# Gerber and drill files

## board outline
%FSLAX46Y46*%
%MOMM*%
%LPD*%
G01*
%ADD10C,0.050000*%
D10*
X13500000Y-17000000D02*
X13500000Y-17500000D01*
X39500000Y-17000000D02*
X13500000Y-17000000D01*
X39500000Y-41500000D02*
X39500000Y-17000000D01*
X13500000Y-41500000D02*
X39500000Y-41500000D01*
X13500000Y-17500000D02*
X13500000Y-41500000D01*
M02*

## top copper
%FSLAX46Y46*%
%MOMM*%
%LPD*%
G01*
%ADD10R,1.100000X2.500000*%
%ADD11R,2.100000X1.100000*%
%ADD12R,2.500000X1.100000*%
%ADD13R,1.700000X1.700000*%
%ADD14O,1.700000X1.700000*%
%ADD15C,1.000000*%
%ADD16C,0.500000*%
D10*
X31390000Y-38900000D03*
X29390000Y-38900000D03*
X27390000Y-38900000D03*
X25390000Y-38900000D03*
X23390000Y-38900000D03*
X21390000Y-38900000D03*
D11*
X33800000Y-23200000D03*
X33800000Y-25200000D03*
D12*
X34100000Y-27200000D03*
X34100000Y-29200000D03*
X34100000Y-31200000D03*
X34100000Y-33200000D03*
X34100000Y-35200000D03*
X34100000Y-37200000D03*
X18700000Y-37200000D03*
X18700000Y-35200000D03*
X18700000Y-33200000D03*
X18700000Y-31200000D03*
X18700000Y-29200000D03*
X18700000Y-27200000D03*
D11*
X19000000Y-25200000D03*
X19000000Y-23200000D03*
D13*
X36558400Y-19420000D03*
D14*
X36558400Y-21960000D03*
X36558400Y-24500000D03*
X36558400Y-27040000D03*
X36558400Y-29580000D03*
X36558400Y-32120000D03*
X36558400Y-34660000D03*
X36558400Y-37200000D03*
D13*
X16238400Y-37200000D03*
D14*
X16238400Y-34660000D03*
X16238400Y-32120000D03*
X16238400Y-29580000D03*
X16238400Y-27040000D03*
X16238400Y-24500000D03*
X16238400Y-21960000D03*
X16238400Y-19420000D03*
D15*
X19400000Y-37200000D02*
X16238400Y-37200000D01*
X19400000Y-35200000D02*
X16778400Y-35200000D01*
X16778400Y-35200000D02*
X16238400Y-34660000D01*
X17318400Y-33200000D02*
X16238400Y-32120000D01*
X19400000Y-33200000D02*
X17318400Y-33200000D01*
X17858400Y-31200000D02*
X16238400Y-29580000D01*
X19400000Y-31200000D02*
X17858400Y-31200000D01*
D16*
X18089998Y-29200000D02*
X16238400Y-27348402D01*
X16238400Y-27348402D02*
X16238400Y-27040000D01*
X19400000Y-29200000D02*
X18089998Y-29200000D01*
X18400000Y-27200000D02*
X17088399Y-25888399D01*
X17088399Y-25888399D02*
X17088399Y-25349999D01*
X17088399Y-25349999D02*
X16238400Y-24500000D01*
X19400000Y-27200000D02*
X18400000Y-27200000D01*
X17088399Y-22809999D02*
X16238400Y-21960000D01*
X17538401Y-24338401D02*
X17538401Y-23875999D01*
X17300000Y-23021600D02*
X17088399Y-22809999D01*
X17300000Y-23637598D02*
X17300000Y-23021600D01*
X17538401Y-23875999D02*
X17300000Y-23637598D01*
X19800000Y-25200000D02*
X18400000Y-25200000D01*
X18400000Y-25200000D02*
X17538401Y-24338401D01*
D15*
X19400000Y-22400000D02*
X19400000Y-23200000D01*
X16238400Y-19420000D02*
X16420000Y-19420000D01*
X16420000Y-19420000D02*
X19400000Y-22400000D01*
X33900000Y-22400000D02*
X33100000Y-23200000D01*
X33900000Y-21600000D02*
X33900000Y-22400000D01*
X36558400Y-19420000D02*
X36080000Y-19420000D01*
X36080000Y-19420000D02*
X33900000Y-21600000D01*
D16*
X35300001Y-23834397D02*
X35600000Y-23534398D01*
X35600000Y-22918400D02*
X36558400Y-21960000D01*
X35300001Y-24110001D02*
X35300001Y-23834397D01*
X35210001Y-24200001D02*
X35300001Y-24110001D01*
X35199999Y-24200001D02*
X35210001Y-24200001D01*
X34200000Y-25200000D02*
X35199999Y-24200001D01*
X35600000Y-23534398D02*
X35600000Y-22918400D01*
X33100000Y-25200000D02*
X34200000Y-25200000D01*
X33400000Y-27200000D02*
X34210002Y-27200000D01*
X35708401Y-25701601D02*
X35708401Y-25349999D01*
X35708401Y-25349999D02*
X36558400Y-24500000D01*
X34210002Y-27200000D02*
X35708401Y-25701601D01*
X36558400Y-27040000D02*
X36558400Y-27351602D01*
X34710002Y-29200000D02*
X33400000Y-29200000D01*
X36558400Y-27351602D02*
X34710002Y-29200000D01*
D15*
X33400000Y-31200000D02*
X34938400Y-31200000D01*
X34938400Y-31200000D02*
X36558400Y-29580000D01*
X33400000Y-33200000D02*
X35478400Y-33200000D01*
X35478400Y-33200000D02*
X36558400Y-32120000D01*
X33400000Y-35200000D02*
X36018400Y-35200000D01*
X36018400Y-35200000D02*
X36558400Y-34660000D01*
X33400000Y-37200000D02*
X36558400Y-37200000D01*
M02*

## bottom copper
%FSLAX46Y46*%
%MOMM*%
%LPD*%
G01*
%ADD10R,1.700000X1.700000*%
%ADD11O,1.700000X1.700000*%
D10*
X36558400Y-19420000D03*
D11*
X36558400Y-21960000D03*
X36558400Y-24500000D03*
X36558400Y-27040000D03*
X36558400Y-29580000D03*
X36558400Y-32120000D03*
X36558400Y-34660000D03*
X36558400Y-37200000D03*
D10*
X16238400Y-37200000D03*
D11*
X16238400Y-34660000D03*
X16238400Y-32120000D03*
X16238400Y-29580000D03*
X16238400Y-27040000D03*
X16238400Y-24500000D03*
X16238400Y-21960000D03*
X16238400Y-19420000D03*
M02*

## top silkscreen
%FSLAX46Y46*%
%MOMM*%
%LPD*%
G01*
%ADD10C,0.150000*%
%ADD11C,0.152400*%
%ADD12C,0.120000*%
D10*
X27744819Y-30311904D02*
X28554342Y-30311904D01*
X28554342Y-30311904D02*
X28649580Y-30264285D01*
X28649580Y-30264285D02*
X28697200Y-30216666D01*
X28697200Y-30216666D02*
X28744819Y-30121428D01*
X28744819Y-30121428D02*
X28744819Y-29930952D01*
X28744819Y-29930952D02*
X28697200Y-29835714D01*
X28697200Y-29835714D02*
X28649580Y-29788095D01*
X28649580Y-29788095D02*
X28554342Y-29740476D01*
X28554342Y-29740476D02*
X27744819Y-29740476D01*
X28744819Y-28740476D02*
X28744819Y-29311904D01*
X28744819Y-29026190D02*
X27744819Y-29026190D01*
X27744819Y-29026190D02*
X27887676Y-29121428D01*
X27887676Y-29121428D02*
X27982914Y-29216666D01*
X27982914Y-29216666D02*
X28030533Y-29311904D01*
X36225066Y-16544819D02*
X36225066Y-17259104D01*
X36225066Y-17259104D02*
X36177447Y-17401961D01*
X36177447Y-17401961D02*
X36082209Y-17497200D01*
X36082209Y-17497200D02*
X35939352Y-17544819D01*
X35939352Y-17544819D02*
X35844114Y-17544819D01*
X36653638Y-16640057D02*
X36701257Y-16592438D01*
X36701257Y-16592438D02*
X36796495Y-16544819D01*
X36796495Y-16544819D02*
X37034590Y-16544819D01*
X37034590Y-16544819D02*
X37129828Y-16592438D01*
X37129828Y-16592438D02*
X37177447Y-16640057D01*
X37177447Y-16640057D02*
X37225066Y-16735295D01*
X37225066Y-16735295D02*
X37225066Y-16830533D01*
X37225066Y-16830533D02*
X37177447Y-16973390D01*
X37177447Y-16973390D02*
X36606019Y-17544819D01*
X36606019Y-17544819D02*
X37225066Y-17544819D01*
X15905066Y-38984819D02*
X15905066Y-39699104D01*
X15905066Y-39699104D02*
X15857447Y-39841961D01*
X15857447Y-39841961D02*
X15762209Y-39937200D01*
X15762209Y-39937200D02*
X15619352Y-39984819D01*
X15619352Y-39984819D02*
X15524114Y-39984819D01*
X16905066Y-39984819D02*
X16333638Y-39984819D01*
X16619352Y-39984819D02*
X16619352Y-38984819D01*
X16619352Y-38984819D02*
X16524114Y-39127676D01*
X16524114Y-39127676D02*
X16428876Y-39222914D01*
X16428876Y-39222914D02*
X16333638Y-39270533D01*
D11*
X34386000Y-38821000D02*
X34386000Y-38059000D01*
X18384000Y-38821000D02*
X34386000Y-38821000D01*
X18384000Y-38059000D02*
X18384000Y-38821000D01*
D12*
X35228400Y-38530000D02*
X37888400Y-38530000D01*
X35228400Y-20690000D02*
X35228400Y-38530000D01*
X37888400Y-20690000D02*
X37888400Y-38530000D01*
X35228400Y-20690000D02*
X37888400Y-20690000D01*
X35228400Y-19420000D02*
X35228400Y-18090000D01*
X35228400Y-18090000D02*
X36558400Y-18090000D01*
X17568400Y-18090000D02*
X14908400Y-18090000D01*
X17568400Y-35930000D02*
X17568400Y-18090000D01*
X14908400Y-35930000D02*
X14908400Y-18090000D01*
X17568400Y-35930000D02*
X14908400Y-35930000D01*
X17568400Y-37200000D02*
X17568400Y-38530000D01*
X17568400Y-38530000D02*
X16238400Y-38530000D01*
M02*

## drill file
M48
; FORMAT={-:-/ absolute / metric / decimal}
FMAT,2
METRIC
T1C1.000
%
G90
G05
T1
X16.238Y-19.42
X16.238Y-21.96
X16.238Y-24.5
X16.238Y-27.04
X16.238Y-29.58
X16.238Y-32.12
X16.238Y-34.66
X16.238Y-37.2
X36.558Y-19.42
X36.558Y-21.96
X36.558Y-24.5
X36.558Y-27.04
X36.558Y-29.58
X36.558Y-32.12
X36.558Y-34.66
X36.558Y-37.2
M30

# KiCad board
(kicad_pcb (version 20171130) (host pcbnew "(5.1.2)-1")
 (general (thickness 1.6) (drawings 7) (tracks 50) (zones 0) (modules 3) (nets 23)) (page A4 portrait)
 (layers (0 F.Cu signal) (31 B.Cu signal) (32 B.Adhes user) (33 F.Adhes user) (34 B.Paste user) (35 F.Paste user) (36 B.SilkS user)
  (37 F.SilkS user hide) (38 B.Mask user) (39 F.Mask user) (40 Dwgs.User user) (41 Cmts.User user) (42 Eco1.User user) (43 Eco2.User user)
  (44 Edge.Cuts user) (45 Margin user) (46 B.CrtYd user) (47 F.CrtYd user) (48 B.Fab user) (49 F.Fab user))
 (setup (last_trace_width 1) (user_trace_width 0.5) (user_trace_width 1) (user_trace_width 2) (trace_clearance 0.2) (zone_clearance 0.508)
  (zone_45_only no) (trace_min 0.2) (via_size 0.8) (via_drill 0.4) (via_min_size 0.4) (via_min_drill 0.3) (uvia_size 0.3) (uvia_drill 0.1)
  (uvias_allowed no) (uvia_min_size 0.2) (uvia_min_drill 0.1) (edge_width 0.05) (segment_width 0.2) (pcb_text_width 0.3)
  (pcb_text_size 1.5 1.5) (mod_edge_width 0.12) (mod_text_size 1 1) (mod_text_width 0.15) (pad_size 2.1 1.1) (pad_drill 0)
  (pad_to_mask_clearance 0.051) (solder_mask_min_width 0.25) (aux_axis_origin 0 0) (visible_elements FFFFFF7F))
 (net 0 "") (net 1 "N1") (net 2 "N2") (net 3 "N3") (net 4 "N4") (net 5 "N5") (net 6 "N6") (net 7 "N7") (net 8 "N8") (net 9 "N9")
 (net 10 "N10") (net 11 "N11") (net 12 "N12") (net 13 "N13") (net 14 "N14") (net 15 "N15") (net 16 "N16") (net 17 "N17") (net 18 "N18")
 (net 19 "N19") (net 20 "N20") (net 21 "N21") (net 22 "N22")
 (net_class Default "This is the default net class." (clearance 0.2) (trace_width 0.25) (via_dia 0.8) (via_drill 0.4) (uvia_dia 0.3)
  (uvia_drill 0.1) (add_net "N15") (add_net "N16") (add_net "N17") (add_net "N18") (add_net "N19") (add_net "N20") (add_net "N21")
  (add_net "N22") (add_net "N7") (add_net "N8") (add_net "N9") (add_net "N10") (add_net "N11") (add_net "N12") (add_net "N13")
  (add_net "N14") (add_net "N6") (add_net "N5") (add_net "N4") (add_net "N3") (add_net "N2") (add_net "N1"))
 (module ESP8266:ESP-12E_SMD (layer F.Cu) (at 19.4 23.2)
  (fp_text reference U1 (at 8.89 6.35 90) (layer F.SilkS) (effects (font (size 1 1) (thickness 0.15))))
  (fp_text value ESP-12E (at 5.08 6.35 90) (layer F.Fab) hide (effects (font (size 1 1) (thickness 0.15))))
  (fp_line (start 14.986 15.621) (end 14.986 14.859) (layer F.SilkS) (width 0.1524))
  (fp_line (start -1.016 15.621) (end 14.986 15.621) (layer F.SilkS) (width 0.1524))
  (fp_line (start -1.016 14.859) (end -1.016 15.621) (layer F.SilkS) (width 0.1524))
  (pad 22 smd rect (at 11.99 15 90) (size 2.5 1.1) (drill (offset -0.7 0)) (layers F.Cu F.Paste F.Mask) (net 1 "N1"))
  (pad 21 smd rect (at 9.99 15 90) (size 2.5 1.1) (drill (offset -0.7 0)) (layers F.Cu F.Paste F.Mask) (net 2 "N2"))
  (pad 20 smd rect (at 7.99 15 90) (size 2.5 1.1) (drill (offset -0.7 0)) (layers F.Cu F.Paste F.Mask) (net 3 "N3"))
  (pad 19 smd rect (at 5.99 15 90) (size 2.5 1.1) (drill (offset -0.7 0)) (layers F.Cu F.Paste F.Mask) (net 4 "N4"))
  (pad 18 smd rect (at 3.99 15 90) (size 2.5 1.1) (drill (offset -0.7 0)) (layers F.Cu F.Paste F.Mask) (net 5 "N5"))
  (pad 17 smd rect (at 1.99 15 90) (size 2.5 1.1) (drill (offset -0.7 0)) (layers F.Cu F.Paste F.Mask) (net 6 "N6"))
  (pad 16 smd rect (at 13.7 0) (size 2.1 1.1) (drill (offset 0.7 0)) (layers F.Cu F.Paste F.Mask) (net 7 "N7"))
  (pad 15 smd rect (at 13.7 2) (size 2.1 1.1) (drill (offset 0.7 0)) (layers F.Cu F.Paste F.Mask) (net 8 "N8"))
  (pad 14 smd rect (at 14 4) (size 2.5 1.1) (drill (offset 0.7 0)) (layers F.Cu F.Paste F.Mask) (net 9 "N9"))
  (pad 13 smd rect (at 14 6) (size 2.5 1.1) (drill (offset 0.7 0)) (layers F.Cu F.Paste F.Mask) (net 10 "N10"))
  (pad 12 smd rect (at 14 8) (size 2.5 1.1) (drill (offset 0.7 0)) (layers F.Cu F.Paste F.Mask) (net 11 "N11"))
  (pad 11 smd rect (at 14 10) (size 2.5 1.1) (drill (offset 0.7 0)) (layers F.Cu F.Paste F.Mask) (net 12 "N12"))
  (pad 10 smd rect (at 14 12) (size 2.5 1.1) (drill (offset 0.7 0)) (layers F.Cu F.Paste F.Mask) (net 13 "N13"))
  (pad 9 smd rect (at 14 14) (size 2.5 1.1) (drill (offset 0.7 0)) (layers F.Cu F.Paste F.Mask) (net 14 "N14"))
  (pad 8 smd rect (at 0 14) (size 2.5 1.1) (drill (offset -0.7 0)) (layers F.Cu F.Paste F.Mask) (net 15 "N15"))
  (pad 7 smd rect (at 0 12) (size 2.5 1.1) (drill (offset -0.7 0)) (layers F.Cu F.Paste F.Mask) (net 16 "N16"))
  (pad 6 smd rect (at 0 10) (size 2.5 1.1) (drill (offset -0.7 0)) (layers F.Cu F.Paste F.Mask) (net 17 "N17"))
  (pad 5 smd rect (at 0 8) (size 2.5 1.1) (drill (offset -0.7 0)) (layers F.Cu F.Paste F.Mask) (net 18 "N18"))
  (pad 4 smd rect (at 0 6) (size 2.5 1.1) (drill (offset -0.7 0)) (layers F.Cu F.Paste F.Mask) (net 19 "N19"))
  (pad 3 smd rect (at 0 4) (size 2.5 1.1) (drill (offset -0.7 0)) (layers F.Cu F.Paste F.Mask) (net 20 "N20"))
  (pad 2 smd rect (at 0.3 2) (size 2.1 1.1) (drill (offset -0.7 0)) (layers F.Cu F.Paste F.Mask) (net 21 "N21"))
  (pad 1 smd rect (at 0.3 0) (size 2.1 1.1) (drill (offset -0.7 0)) (layers F.Cu F.Paste F.Mask) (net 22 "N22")))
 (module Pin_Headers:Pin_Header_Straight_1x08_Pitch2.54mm (layer F.Cu) (at 36.5584 19.42)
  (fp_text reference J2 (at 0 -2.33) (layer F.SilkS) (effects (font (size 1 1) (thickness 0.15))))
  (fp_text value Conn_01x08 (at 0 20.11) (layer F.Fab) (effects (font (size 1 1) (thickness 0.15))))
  (fp_line (start -1.33 19.11) (end 1.33 19.11) (layer F.SilkS) (width 0.12))
  (fp_line (start -1.33 1.27) (end -1.33 19.11) (layer F.SilkS) (width 0.12))
  (fp_line (start 1.33 1.27) (end 1.33 19.11) (layer F.SilkS) (width 0.12))
  (fp_line (start -1.33 1.27) (end 1.33 1.27) (layer F.SilkS) (width 0.12))
  (fp_line (start -1.33 0) (end -1.33 -1.33) (layer F.SilkS) (width 0.12))
  (fp_line (start -1.33 -1.33) (end 0 -1.33) (layer F.SilkS) (width 0.12))
  (pad 1 thru_hole rect (at 0 0) (size 1.7 1.7) (drill 1) (layers *.Cu *.Mask) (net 7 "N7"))
  (pad 2 thru_hole oval (at 0 2.54) (size 1.7 1.7) (drill 1) (layers *.Cu *.Mask) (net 8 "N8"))
  (pad 3 thru_hole oval (at 0 5.08) (size 1.7 1.7) (drill 1) (layers *.Cu *.Mask) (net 9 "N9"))
  (pad 4 thru_hole oval (at 0 7.62) (size 1.7 1.7) (drill 1) (layers *.Cu *.Mask) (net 10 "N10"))
  (pad 5 thru_hole oval (at 0 10.16) (size 1.7 1.7) (drill 1) (layers *.Cu *.Mask) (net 11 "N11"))
  (pad 6 thru_hole oval (at 0 12.7) (size 1.7 1.7) (drill 1) (layers *.Cu *.Mask) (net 12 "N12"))
  (pad 7 thru_hole oval (at 0 15.24) (size 1.7 1.7) (drill 1) (layers *.Cu *.Mask) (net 13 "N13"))
  (pad 8 thru_hole oval (at 0 17.78) (size 1.7 1.7) (drill 1) (layers *.Cu *.Mask) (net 14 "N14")))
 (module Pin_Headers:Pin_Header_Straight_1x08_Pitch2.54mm (layer F.Cu) (at 16.2384 37.2 180)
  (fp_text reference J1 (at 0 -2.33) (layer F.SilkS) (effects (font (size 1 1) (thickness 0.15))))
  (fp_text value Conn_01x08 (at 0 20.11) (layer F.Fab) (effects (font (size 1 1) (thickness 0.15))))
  (fp_line (start -1.33 19.11) (end 1.33 19.11) (layer F.SilkS) (width 0.12))
  (fp_line (start -1.33 1.27) (end -1.33 19.11) (layer F.SilkS) (width 0.12))
  (fp_line (start 1.33 1.27) (end 1.33 19.11) (layer F.SilkS) (width 0.12))
  (fp_line (start -1.33 1.27) (end 1.33 1.27) (layer F.SilkS) (width 0.12))
  (fp_line (start -1.33 0) (end -1.33 -1.33) (layer F.SilkS) (width 0.12))
  (fp_line (start -1.33 -1.33) (end 0 -1.33) (layer F.SilkS) (width 0.12))
  (pad 1 thru_hole rect (at 0 0 180) (size 1.7 1.7) (drill 1) (layers *.Cu *.Mask) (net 15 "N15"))
  (pad 2 thru_hole oval (at 0 2.54 180) (size 1.7 1.7) (drill 1) (layers *.Cu *.Mask) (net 16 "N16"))
  (pad 3 thru_hole oval (at 0 5.08 180) (size 1.7 1.7) (drill 1) (layers *.Cu *.Mask) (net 17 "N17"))
  (pad 4 thru_hole oval (at 0 7.62 180) (size 1.7 1.7) (drill 1) (layers *.Cu *.Mask) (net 18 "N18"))
  (pad 5 thru_hole oval (at 0 10.16 180) (size 1.7 1.7) (drill 1) (layers *.Cu *.Mask) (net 19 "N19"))
  (pad 6 thru_hole oval (at 0 12.7 180) (size 1.7 1.7) (drill 1) (layers *.Cu *.Mask) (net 20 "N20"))
  (pad 7 thru_hole oval (at 0 15.24 180) (size 1.7 1.7) (drill 1) (layers *.Cu *.Mask) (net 21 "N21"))
  (pad 8 thru_hole oval (at 0 17.78 180) (size 1.7 1.7) (drill 1) (layers *.Cu *.Mask) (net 22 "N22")))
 (gr_line (start 13.5 17) (end 13.5 17.5) (layer Edge.Cuts) (width 0.05))
 (gr_line (start 39.5 17) (end 13.5 17) (layer Edge.Cuts) (width 0.05))
 (gr_line (start 39.5 41.5) (end 39.5 17) (layer Edge.Cuts) (width 0.05))
 (gr_line (start 13.5 41.5) (end 39.5 41.5) (layer Edge.Cuts) (width 0.05))
 (gr_line (start 13.5 17.5) (end 13.5 41.5) (layer Edge.Cuts) (width 0.05))
 (segment (start 19.4 37.2) (end 16.2384 37.2) (width 1) (layer F.Cu) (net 15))
 (segment (start 19.4 35.2) (end 16.7784 35.2) (width 1) (layer F.Cu) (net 16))
 (segment (start 16.7784 35.2) (end 16.2384 34.66) (width 1) (layer F.Cu) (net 16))
 (segment (start 17.3184 33.2) (end 16.2384 32.12) (width 1) (layer F.Cu) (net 17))
 (segment (start 19.4 33.2) (end 17.3184 33.2) (width 1) (layer F.Cu) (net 17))
 (segment (start 17.8584 31.2) (end 16.2384 29.58) (width 1) (layer F.Cu) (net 18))
 (segment (start 19.4 31.2) (end 17.8584 31.2) (width 1) (layer F.Cu) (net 18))
 (segment (start 18.089998 29.2) (end 16.2384 27.348402) (width 0.5) (layer F.Cu) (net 19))
 (segment (start 16.2384 27.348402) (end 16.2384 27.04) (width 0.5) (layer F.Cu) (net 19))
 (segment (start 19.4 29.2) (end 18.089998 29.2) (width 0.5) (layer F.Cu) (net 19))
 (segment (start 18.4 27.2) (end 17.088399 25.888399) (width 0.5) (layer F.Cu) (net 20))
 (segment (start 17.088399 25.888399) (end 17.088399 25.349999) (width 0.5) (layer F.Cu) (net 20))
 (segment (start 17.088399 25.349999) (end 16.2384 24.5) (width 0.5) (layer F.Cu) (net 20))
 (segment (start 19.4 27.2) (end 18.4 27.2) (width 0.5) (layer F.Cu) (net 20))
 (segment (start 17.088399 22.809999) (end 16.2384 21.96) (width 0.5) (layer F.Cu) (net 21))
 (segment (start 17.538401 24.338401) (end 17.538401 23.875999) (width 0.5) (layer F.Cu) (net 21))
 (segment (start 17.3 23.0216) (end 17.088399 22.809999) (width 0.5) (layer F.Cu) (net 21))
 (segment (start 17.3 23.637598) (end 17.3 23.0216) (width 0.5) (layer F.Cu) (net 21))
 (segment (start 17.538401 23.875999) (end 17.3 23.637598) (width 0.5) (layer F.Cu) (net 21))
 (segment (start 19.8 25.2) (end 18.4 25.2) (width 0.5) (layer F.Cu) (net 21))
 (segment (start 18.4 25.2) (end 17.538401 24.338401) (width 0.5) (layer F.Cu) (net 21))
 (segment (start 19.4 22.4) (end 19.4 23.2) (width 1) (layer F.Cu) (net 22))
 (segment (start 16.2384 19.42) (end 16.42 19.42) (width 1) (layer F.Cu) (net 22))
 (segment (start 16.42 19.42) (end 19.4 22.4) (width 1) (layer F.Cu) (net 22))
 (segment (start 33.9 22.4) (end 33.1 23.2) (width 1) (layer F.Cu) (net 7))
 (segment (start 33.9 21.6) (end 33.9 22.4) (width 1) (layer F.Cu) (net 7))
 (segment (start 36.5584 19.42) (end 36.08 19.42) (width 1) (layer F.Cu) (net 7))
 (segment (start 36.08 19.42) (end 33.9 21.6) (width 1) (layer F.Cu) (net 7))
 (segment (start 35.300001 23.834397) (end 35.6 23.534398) (width 0.5) (layer F.Cu) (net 8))
 (segment (start 35.6 22.9184) (end 36.5584 21.96) (width 0.5) (layer F.Cu) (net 8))
 (segment (start 35.300001 24.110001) (end 35.300001 23.834397) (width 0.5) (layer F.Cu) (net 8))
 (segment (start 35.210001 24.200001) (end 35.300001 24.110001) (width 0.5) (layer F.Cu) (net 8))
 (segment (start 35.199999 24.200001) (end 35.210001 24.200001) (width 0.5) (layer F.Cu) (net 8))
 (segment (start 34.2 25.2) (end 35.199999 24.200001) (width 0.5) (layer F.Cu) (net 8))
 (segment (start 35.6 23.534398) (end 35.6 22.9184) (width 0.5) (layer F.Cu) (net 8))
 (segment (start 33.1 25.2) (end 34.2 25.2) (width 0.5) (layer F.Cu) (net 8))
 (segment (start 33.4 27.2) (end 34.210002 27.2) (width 0.5) (layer F.Cu) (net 9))
 (segment (start 35.708401 25.701601) (end 35.708401 25.349999) (width 0.5) (layer F.Cu) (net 9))
 (segment (start 35.708401 25.349999) (end 36.5584 24.5) (width 0.5) (layer F.Cu) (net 9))
 (segment (start 34.210002 27.2) (end 35.708401 25.701601) (width 0.5) (layer F.Cu) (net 9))
 (segment (start 36.5584 27.04) (end 36.5584 27.351602) (width 0.5) (layer F.Cu) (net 10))
 (segment (start 34.710002 29.2) (end 33.4 29.2) (width 0.5) (layer F.Cu) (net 10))
 (segment (start 36.5584 27.351602) (end 34.710002 29.2) (width 0.5) (layer F.Cu) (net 10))
 (segment (start 33.4 31.2) (end 34.9384 31.2) (width 1) (layer F.Cu) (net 11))
 (segment (start 34.9384 31.2) (end 36.5584 29.58) (width 1) (layer F.Cu) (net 11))
 (segment (start 33.4 33.2) (end 35.4784 33.2) (width 1) (layer F.Cu) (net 12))
 (segment (start 35.4784 33.2) (end 36.5584 32.12) (width 1) (layer F.Cu) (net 12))
 (segment (start 33.4 35.2) (end 36.0184 35.2) (width 1) (layer F.Cu) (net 13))
 (segment (start 36.0184 35.2) (end 36.5584 34.66) (width 1) (layer F.Cu) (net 13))
 (segment (start 33.4 37.2) (end 36.5584 37.2) (width 1) (layer F.Cu) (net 14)))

